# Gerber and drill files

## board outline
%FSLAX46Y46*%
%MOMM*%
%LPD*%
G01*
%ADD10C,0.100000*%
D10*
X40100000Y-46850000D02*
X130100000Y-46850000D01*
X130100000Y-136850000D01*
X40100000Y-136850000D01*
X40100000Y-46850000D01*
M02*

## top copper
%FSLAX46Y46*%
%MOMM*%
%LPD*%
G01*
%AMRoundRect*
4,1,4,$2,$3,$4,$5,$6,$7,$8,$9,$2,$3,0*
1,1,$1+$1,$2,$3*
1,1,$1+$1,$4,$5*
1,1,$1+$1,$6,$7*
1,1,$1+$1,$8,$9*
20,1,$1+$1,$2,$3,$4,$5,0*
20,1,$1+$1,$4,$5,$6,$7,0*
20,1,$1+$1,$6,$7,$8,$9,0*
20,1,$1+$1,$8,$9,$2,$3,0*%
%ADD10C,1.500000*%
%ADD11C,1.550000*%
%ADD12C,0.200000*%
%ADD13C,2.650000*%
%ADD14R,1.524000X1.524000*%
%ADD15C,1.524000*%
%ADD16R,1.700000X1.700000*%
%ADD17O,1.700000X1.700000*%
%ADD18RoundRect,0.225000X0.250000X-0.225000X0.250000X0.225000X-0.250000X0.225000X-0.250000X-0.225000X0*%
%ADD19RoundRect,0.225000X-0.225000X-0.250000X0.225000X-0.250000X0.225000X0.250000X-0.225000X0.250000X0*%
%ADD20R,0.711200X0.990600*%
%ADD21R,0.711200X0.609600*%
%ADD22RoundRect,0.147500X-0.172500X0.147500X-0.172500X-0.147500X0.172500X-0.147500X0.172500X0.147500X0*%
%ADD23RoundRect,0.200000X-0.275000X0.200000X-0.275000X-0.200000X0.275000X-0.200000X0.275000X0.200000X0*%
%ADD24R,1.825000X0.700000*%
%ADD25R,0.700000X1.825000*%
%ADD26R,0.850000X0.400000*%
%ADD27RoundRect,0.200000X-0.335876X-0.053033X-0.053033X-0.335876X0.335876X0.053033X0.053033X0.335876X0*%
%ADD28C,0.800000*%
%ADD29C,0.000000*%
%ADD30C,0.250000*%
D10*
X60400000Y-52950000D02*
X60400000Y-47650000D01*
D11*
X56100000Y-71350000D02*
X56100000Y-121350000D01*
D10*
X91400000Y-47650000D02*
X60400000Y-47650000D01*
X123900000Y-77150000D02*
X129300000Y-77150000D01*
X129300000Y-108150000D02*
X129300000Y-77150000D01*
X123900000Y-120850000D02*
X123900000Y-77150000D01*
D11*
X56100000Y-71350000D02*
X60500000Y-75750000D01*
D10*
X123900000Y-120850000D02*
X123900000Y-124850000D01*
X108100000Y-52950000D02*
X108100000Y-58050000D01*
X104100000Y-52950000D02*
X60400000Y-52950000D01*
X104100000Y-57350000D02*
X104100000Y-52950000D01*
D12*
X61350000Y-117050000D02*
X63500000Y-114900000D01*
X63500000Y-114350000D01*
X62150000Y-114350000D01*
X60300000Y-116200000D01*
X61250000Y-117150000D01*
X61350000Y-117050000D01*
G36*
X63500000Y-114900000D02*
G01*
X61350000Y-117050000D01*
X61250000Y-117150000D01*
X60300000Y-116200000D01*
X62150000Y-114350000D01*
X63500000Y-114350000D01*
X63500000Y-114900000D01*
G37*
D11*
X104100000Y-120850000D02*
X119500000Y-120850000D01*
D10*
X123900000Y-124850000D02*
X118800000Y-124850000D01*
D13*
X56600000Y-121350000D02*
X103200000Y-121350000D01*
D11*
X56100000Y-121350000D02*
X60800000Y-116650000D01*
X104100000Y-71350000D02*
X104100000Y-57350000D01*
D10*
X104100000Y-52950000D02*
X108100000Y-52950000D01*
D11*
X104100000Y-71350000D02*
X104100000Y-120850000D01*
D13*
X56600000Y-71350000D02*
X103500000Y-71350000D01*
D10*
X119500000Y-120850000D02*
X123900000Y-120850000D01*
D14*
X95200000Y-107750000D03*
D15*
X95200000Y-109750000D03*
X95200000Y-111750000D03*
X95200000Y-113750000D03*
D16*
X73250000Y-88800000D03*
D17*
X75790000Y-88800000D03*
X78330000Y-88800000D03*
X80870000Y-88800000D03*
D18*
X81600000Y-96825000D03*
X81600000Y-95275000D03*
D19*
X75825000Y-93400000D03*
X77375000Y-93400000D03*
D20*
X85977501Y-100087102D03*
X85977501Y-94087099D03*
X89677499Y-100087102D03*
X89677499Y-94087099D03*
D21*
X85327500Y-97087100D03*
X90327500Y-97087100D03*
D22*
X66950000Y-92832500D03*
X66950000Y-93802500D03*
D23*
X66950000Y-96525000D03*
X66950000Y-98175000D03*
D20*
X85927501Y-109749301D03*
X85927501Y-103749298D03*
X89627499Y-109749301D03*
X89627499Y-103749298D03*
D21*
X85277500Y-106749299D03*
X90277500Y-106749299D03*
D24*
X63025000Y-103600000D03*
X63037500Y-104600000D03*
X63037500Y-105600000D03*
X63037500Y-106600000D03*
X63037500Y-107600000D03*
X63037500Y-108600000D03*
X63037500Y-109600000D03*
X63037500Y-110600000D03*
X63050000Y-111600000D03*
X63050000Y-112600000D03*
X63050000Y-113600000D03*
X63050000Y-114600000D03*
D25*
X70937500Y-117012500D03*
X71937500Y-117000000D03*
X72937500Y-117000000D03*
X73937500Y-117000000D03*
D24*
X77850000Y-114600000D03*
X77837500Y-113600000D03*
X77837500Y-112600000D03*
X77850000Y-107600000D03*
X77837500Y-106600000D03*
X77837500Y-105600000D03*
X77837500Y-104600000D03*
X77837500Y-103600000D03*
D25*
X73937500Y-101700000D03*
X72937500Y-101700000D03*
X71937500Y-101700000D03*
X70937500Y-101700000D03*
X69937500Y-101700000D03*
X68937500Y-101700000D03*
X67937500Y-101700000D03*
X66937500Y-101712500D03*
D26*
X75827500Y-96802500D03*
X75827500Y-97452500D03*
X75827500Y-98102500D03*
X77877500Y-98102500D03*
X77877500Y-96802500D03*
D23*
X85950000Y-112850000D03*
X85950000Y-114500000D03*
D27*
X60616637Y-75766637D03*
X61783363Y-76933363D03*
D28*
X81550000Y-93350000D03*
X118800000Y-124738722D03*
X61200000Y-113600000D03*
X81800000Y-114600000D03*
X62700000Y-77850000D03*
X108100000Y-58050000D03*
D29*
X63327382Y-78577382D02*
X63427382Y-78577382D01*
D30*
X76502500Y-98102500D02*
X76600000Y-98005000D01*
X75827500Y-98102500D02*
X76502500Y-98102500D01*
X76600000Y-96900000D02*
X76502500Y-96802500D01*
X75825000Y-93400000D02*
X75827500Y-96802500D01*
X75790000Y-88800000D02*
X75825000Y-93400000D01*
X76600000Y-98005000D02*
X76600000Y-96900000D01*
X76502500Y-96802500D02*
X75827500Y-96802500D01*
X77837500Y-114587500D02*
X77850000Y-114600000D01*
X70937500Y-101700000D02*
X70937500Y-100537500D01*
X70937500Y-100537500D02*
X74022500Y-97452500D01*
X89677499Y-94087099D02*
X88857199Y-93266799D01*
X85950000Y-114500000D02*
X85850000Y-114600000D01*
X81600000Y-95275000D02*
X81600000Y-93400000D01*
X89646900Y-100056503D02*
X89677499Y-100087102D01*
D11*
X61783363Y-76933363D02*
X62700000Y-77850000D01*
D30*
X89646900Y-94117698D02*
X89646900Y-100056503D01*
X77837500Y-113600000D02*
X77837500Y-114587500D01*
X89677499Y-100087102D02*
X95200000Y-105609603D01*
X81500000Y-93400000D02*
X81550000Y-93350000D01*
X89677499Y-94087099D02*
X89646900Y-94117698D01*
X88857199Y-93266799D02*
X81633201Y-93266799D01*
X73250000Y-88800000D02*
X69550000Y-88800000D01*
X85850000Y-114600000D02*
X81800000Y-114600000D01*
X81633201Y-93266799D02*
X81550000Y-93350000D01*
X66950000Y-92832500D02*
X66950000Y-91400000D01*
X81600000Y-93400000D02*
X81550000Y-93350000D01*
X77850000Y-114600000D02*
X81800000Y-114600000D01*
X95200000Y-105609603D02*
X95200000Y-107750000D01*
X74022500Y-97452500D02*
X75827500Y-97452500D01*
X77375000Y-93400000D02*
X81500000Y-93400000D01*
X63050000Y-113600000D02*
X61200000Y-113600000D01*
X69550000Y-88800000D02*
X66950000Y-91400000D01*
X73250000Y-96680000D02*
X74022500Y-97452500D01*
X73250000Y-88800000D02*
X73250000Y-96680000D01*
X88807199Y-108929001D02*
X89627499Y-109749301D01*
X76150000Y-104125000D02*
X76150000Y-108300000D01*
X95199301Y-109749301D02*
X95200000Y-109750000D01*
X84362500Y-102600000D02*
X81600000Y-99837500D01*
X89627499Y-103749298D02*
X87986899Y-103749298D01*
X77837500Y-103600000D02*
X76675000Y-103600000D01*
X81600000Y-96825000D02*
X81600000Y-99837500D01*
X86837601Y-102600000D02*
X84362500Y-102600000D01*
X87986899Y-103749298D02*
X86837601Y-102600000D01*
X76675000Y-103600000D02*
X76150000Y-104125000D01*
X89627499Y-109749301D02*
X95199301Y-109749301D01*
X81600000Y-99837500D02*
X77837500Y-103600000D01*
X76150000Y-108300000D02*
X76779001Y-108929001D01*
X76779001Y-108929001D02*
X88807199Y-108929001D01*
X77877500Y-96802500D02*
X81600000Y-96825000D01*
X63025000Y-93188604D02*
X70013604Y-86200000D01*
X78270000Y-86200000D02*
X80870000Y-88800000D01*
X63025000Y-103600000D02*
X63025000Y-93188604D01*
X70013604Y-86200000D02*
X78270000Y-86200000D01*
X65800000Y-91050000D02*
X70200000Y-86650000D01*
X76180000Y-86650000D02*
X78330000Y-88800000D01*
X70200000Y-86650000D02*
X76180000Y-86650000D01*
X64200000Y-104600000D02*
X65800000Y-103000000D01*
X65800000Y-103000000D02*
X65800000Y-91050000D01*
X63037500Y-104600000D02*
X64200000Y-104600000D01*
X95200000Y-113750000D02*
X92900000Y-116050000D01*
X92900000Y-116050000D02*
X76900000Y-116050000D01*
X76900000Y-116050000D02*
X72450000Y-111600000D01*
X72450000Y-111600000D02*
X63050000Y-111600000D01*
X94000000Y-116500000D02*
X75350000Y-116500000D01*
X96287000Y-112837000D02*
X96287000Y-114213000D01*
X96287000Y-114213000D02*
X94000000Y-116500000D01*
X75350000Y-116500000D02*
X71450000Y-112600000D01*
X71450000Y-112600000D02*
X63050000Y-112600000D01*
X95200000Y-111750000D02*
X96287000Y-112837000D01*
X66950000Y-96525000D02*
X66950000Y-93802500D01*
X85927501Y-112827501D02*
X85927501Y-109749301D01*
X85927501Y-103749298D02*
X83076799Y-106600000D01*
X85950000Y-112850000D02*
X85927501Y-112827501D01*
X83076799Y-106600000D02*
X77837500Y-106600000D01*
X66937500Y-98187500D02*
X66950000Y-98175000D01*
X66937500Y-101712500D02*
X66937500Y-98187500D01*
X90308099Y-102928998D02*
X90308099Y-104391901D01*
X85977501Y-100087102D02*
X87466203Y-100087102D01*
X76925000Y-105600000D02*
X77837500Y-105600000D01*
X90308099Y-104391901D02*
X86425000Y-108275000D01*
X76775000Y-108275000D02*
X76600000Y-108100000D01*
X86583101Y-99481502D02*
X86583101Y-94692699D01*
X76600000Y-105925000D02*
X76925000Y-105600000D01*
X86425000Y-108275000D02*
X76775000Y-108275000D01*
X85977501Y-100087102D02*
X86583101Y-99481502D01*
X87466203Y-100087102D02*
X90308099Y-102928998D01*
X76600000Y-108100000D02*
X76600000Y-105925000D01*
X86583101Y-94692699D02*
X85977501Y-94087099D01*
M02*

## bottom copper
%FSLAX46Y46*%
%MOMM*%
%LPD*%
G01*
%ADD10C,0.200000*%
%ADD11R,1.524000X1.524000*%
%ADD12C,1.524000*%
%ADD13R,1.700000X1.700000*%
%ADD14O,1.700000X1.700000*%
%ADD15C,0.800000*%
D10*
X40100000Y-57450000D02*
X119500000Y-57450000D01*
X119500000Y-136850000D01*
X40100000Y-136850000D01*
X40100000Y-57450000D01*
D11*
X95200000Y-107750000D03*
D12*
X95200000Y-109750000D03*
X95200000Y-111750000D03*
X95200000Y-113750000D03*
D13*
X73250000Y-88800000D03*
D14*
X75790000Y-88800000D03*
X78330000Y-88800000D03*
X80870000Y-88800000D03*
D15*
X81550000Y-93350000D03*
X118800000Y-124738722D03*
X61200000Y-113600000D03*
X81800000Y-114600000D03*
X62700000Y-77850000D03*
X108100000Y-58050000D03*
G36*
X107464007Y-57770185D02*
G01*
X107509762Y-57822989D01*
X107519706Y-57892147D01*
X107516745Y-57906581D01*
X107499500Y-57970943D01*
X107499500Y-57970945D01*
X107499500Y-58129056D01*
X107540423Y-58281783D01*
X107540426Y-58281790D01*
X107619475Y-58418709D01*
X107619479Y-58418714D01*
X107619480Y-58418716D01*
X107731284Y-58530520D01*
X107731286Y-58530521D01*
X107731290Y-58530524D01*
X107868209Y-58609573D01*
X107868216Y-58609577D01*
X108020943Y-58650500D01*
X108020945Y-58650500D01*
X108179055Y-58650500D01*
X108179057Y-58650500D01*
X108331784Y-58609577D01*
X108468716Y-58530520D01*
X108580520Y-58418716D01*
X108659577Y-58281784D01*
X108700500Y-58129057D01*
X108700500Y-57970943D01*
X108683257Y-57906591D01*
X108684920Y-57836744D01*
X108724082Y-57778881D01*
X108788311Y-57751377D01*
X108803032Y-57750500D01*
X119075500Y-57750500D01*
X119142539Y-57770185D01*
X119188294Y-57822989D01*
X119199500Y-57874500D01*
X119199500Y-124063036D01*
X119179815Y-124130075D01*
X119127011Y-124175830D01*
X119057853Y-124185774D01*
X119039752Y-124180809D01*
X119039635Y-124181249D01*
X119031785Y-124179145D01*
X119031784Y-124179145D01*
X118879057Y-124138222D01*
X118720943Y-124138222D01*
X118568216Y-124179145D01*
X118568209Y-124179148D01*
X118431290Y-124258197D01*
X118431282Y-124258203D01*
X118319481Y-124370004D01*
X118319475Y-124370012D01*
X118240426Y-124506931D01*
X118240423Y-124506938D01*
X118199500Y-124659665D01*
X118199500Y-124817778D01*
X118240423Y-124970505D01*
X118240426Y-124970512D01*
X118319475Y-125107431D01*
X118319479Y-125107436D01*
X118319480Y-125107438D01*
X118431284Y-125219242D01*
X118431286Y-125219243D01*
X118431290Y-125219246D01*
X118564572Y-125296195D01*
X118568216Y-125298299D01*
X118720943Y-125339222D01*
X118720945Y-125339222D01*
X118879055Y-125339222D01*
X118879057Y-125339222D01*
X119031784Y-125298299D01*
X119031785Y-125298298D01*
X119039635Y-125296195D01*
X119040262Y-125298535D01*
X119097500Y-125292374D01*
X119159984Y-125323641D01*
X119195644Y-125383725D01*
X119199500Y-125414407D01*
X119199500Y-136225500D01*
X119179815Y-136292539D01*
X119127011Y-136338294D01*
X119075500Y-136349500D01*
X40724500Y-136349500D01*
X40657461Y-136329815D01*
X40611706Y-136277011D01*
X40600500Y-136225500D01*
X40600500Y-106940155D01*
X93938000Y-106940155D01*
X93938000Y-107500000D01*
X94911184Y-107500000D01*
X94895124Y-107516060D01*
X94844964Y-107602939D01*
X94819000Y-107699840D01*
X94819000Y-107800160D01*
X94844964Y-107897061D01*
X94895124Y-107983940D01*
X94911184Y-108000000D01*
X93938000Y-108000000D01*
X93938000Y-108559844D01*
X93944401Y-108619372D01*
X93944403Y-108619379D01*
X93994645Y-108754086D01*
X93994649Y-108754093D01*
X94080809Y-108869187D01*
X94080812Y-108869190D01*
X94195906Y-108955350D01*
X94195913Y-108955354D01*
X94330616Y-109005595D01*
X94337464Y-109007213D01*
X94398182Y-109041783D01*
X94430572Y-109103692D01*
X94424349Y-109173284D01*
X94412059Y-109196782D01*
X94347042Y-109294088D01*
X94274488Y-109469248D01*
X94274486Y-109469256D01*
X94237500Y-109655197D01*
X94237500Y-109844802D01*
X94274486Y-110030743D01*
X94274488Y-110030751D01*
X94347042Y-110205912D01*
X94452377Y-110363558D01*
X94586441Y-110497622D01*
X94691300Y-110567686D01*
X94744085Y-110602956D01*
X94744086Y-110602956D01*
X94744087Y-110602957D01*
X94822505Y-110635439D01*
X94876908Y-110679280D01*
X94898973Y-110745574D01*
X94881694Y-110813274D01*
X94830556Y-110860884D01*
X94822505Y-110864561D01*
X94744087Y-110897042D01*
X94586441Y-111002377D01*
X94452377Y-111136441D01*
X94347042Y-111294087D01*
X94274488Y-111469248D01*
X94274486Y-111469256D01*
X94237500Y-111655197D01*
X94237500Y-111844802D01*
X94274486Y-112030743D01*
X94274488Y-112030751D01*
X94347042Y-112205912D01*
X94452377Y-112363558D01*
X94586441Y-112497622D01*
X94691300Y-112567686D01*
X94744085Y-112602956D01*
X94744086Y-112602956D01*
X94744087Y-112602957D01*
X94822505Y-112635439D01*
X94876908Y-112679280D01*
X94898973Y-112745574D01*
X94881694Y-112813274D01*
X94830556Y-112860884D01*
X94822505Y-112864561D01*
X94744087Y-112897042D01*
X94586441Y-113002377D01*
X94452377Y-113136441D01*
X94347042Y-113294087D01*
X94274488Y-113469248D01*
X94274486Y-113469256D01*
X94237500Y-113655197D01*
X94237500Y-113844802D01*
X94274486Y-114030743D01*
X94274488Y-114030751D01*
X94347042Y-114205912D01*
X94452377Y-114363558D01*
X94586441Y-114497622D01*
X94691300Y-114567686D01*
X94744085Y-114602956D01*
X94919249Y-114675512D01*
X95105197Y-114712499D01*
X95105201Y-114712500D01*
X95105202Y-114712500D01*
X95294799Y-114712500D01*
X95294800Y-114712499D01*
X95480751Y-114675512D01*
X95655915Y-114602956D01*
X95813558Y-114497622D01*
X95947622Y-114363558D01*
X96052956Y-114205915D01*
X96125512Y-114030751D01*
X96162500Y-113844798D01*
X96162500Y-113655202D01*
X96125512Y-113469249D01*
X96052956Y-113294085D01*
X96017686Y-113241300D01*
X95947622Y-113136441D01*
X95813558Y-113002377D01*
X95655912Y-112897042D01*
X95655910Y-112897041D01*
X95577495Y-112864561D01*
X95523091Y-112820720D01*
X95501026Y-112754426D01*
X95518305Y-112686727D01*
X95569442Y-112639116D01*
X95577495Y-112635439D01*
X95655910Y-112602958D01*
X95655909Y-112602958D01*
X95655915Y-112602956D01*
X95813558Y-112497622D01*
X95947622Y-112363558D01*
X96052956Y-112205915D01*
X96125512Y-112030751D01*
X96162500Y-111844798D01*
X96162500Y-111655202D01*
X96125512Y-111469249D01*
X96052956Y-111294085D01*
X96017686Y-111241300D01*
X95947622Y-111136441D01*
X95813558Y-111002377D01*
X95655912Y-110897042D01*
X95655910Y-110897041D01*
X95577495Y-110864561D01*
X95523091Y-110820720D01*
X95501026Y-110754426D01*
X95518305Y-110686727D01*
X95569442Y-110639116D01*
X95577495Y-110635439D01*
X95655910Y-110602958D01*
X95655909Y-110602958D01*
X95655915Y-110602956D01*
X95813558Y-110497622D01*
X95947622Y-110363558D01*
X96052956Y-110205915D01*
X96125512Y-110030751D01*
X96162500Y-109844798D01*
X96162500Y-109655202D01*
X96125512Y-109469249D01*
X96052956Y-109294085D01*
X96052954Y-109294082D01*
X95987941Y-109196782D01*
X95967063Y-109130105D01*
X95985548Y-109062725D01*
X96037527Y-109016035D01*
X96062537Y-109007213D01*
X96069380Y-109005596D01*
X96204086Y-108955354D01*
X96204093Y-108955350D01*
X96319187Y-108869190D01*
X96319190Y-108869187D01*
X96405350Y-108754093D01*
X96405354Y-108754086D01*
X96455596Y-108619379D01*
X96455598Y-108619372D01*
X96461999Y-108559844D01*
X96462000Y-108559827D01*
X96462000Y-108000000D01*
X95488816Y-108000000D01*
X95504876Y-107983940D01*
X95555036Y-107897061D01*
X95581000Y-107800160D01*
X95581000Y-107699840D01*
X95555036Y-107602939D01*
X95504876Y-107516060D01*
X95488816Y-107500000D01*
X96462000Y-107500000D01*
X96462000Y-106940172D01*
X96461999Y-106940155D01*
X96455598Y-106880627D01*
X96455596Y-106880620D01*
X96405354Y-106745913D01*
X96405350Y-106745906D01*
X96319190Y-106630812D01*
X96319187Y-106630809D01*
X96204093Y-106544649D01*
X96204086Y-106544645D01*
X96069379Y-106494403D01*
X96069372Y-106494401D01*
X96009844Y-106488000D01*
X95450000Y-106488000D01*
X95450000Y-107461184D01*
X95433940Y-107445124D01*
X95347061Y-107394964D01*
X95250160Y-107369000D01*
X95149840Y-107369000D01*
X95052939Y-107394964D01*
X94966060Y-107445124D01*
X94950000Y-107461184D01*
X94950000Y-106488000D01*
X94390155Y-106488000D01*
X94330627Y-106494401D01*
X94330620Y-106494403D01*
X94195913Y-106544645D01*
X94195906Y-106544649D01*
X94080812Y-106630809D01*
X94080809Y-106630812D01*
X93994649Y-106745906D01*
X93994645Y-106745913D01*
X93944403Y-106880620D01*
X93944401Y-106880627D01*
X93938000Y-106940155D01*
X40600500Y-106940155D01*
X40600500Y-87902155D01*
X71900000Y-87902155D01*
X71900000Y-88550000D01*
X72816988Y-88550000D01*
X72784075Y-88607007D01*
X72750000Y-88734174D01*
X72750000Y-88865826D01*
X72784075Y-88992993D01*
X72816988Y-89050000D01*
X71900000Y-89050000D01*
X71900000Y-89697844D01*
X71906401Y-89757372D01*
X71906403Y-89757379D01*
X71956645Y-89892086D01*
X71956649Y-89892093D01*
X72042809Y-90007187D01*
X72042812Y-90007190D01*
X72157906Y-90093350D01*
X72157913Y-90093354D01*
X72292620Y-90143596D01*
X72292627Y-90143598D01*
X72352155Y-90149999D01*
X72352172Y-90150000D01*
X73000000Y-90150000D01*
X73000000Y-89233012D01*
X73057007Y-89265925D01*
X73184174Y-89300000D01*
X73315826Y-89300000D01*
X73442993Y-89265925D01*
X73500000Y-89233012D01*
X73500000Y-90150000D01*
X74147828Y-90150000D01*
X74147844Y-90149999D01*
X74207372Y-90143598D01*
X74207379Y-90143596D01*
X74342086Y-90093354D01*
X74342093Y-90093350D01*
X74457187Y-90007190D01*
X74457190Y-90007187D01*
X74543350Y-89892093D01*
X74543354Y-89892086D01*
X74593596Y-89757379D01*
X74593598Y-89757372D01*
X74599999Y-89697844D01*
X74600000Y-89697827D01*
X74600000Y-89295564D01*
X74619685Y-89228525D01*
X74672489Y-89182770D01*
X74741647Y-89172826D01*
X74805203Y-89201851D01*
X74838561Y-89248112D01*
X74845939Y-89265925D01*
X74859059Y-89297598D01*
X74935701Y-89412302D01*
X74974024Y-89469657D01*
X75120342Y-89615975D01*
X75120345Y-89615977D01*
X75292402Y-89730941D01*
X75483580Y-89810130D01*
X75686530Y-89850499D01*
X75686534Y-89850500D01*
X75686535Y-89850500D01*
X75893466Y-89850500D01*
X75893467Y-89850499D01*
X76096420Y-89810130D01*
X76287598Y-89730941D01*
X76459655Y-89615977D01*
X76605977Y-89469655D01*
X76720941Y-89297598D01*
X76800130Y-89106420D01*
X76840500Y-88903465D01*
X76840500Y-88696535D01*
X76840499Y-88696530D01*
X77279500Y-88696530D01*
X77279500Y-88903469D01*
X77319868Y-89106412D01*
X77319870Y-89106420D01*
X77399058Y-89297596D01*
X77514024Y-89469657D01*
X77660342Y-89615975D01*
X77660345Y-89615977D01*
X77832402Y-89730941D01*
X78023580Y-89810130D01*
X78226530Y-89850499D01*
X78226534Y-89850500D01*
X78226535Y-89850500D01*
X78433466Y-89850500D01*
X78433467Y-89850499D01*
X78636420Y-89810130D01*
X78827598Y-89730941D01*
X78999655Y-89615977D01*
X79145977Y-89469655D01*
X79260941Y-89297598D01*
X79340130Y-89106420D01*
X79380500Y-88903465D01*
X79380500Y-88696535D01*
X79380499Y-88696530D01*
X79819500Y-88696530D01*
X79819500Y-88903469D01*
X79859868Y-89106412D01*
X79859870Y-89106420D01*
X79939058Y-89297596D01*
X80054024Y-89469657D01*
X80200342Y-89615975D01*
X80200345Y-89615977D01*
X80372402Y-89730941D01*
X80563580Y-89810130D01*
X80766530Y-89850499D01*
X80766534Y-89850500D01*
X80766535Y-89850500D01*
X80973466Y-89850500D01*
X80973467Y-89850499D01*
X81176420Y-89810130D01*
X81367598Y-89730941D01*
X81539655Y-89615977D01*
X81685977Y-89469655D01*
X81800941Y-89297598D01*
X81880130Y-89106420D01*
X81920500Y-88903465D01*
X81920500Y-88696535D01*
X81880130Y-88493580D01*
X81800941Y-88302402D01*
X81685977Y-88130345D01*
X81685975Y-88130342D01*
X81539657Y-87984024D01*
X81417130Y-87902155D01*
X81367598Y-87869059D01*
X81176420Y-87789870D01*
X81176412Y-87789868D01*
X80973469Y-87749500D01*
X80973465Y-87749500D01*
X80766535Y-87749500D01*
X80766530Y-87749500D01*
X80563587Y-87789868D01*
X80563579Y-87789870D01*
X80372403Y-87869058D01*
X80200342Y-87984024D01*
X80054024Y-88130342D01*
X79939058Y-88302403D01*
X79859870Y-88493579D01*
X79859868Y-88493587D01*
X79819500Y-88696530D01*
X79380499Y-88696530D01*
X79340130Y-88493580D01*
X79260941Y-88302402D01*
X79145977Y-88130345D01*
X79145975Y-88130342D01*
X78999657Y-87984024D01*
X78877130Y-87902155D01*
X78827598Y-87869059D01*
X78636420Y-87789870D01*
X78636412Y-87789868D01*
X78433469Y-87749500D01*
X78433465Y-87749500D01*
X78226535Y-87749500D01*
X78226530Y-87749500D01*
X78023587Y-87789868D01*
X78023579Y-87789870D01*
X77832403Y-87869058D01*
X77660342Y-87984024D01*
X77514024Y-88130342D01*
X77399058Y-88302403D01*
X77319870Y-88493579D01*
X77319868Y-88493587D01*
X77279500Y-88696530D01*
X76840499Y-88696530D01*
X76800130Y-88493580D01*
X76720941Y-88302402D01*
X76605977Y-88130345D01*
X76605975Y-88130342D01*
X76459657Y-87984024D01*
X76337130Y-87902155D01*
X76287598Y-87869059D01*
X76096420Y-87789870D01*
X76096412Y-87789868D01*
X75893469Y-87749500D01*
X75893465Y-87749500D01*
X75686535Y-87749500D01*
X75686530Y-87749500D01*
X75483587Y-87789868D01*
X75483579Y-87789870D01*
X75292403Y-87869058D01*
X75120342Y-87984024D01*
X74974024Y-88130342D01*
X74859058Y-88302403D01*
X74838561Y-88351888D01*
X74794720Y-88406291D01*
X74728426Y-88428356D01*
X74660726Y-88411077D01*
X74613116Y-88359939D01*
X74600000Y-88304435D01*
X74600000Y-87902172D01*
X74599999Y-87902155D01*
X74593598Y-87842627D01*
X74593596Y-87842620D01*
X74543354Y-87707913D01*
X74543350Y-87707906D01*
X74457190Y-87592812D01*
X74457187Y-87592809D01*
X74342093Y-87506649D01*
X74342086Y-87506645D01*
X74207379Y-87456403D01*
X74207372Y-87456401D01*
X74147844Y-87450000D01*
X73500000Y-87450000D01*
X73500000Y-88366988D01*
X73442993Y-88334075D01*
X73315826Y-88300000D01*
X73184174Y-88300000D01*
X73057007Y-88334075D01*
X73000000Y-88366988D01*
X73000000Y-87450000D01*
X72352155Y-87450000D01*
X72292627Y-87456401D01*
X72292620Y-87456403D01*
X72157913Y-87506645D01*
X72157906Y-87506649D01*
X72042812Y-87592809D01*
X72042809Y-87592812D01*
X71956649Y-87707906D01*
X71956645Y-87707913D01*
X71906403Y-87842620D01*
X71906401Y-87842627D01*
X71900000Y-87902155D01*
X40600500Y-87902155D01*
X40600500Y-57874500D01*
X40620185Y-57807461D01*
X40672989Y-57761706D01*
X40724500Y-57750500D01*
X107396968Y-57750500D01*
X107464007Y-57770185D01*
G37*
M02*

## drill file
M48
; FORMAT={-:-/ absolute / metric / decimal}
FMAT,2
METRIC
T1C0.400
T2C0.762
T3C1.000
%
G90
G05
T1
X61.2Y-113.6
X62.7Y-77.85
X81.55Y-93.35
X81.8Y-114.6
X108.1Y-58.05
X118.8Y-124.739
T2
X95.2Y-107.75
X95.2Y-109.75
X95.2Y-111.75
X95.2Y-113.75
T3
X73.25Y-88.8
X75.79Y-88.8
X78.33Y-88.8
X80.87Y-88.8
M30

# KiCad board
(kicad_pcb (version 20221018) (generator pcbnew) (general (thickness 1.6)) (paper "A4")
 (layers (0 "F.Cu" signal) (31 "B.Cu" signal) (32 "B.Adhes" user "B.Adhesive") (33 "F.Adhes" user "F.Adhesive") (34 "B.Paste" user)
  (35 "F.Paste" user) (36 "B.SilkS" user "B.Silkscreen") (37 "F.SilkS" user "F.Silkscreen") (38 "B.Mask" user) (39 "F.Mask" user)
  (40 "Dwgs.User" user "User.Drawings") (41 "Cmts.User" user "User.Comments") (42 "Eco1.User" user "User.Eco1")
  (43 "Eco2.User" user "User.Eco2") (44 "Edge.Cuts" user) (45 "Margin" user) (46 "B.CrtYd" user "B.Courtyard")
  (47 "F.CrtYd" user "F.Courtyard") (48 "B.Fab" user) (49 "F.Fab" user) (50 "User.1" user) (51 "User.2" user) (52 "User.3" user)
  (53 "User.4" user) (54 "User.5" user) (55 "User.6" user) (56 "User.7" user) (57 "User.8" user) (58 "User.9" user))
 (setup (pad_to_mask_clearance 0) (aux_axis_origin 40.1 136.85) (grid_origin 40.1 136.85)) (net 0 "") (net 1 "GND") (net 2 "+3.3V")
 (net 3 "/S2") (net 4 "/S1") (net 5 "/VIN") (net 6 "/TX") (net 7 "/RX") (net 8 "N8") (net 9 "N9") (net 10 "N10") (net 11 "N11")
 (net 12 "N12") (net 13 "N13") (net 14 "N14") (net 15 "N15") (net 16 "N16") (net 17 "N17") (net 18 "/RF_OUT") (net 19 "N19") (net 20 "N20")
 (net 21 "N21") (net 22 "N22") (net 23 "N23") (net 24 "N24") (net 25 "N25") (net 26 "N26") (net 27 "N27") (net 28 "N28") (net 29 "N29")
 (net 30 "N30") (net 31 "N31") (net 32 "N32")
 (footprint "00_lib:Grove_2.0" (layer "F.Cu") (at 95.05 110.75)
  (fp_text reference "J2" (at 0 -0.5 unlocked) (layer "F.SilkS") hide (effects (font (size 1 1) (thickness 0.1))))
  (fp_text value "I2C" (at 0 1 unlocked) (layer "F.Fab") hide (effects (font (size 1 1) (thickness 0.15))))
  (pad "1" thru_hole rect (at 0.15 -3) (size 1.524 1.524) (drill 0.762) (layers "*.Cu" "*.Mask") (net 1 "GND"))
  (pad "2" thru_hole circle (at 0.15 -1) (size 1.524 1.524) (drill 0.762) (layers "*.Cu" "*.Mask") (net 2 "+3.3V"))
  (pad "3" thru_hole circle (at 0.15 1) (size 1.524 1.524) (drill 0.762) (layers "*.Cu" "*.Mask") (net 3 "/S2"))
  (pad "4" thru_hole circle (at 0.15 3) (size 1.524 1.524) (drill 0.762) (layers "*.Cu" "*.Mask") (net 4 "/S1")))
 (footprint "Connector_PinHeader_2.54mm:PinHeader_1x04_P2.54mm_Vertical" (layer "F.Cu") (at 73.25 88.8 90)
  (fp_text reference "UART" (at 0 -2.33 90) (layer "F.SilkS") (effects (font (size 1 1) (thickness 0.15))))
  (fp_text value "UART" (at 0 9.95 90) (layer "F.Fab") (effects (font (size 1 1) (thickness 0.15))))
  (pad "1" thru_hole rect (at 0 0 90) (size 1.7 1.7) (drill 1) (layers "*.Cu" "*.Mask") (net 1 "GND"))
  (pad "2" thru_hole oval (at 0 2.54 90) (size 1.7 1.7) (drill 1) (layers "*.Cu" "*.Mask") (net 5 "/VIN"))
  (pad "3" thru_hole oval (at 0 5.08 90) (size 1.7 1.7) (drill 1) (layers "*.Cu" "*.Mask") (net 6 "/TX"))
  (pad "4" thru_hole oval (at 0 7.62 90) (size 1.7 1.7) (drill 1) (layers "*.Cu" "*.Mask") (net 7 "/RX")))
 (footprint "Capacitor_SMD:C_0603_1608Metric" (layer "F.Cu") (at 81.6 96.05 90)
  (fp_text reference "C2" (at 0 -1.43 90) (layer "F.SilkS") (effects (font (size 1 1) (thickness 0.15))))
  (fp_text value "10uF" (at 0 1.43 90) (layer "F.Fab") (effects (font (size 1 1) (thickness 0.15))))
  (pad "1" smd roundrect (at -0.775 0 90) (size 0.9 0.95) (layers "F.Cu" "F.Paste" "F.Mask") (roundrect_rratio 0.25) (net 2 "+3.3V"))
  (pad "2" smd roundrect (at 0.775 0 90) (size 0.9 0.95) (layers "F.Cu" "F.Paste" "F.Mask") (roundrect_rratio 0.25) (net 1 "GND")))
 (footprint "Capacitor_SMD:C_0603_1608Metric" (layer "F.Cu") (at 76.6 93.4)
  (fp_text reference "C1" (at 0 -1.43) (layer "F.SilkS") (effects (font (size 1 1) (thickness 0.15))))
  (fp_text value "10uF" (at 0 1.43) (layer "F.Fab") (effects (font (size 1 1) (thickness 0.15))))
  (pad "1" smd roundrect (at -0.775 0) (size 0.9 0.95) (layers "F.Cu" "F.Paste" "F.Mask") (roundrect_rratio 0.25) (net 5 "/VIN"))
  (pad "2" smd roundrect (at 0.775 0) (size 0.9 0.95) (layers "F.Cu" "F.Paste" "F.Mask") (roundrect_rratio 0.25) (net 1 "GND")))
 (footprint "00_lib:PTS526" (layer "F.Cu") (at 87.7363 97.037801 90)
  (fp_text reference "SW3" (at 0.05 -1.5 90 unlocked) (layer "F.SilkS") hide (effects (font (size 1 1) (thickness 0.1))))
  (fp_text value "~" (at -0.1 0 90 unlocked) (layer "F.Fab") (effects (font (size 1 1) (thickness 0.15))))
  (pad "1" smd rect (at -3.049301 -1.758799 90) (size 0.9906 0.7112) (layers "F.Cu" "F.Paste" "F.Mask") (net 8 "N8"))
  (pad "2" smd rect (at 2.950702 -1.758799 90) (size 0.9906 0.7112) (layers "F.Cu" "F.Paste" "F.Mask") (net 8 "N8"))
  (pad "3" smd rect (at -3.049301 1.941199 90) (size 0.9906 0.7112) (layers "F.Cu" "F.Paste" "F.Mask") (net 1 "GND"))
  (pad "4" smd rect (at 2.950702 1.941199 90) (size 0.9906 0.7112) (layers "F.Cu" "F.Paste" "F.Mask") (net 1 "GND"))
  (pad "5" smd rect (at -0.049299 -2.4088 180) (size 0.7112 0.6096) (layers "F.Cu" "F.Paste" "F.Mask"))
  (pad "6" smd rect (at -0.049299 2.5912 180) (size 0.7112 0.6096) (layers "F.Cu" "F.Paste" "F.Mask")))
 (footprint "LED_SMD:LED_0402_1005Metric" (layer "F.Cu") (at 66.95 93.3175 -90)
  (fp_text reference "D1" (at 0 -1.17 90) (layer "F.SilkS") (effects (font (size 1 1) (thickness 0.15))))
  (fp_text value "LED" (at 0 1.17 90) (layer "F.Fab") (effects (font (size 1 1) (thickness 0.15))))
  (pad "1" smd roundrect (at -0.485 0 270) (size 0.59 0.64) (layers "F.Cu" "F.Paste" "F.Mask") (roundrect_rratio 0.25) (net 1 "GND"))
  (pad "2" smd roundrect (at 0.485 0 270) (size 0.59 0.64) (layers "F.Cu" "F.Paste" "F.Mask") (roundrect_rratio 0.25) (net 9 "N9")))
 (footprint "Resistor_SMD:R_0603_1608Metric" (layer "F.Cu") (at 66.95 97.35 -90)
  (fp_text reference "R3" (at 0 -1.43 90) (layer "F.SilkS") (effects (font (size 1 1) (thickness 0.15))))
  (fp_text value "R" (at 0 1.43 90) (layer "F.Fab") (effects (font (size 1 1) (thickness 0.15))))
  (pad "1" smd roundrect (at -0.825 0 270) (size 0.8 0.95) (layers "F.Cu" "F.Paste" "F.Mask") (roundrect_rratio 0.25) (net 9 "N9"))
  (pad "2" smd roundrect (at 0.825 0 270) (size 0.8 0.95) (layers "F.Cu" "F.Paste" "F.Mask") (roundrect_rratio 0.25) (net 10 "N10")))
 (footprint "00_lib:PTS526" (layer "F.Cu") (at 87.6863 106.7 90)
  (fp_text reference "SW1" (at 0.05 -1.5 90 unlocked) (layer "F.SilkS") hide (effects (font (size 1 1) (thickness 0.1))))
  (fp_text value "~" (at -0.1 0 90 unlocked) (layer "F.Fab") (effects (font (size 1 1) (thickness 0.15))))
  (pad "1" smd rect (at -3.049301 -1.758799 90) (size 0.9906 0.7112) (layers "F.Cu" "F.Paste" "F.Mask") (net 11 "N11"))
  (pad "2" smd rect (at 2.950702 -1.758799 90) (size 0.9906 0.7112) (layers "F.Cu" "F.Paste" "F.Mask") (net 11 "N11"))
  (pad "3" smd rect (at -3.049301 1.941199 90) (size 0.9906 0.7112) (layers "F.Cu" "F.Paste" "F.Mask") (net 2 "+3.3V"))
  (pad "4" smd rect (at 2.950702 1.941199 90) (size 0.9906 0.7112) (layers "F.Cu" "F.Paste" "F.Mask") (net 2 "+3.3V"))
  (pad "5" smd rect (at -0.049299 -2.4088 180) (size 0.7112 0.6096) (layers "F.Cu" "F.Paste" "F.Mask"))
  (pad "6" smd rect (at -0.049299 2.5912 180) (size 0.7112 0.6096) (layers "F.Cu" "F.Paste" "F.Mask")))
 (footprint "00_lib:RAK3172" (layer "F.Cu") (at 70.4875 109.35 90)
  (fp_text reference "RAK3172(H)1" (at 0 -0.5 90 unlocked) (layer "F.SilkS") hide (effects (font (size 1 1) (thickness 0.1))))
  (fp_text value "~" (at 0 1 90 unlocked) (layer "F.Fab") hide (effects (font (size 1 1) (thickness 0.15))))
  (pad "1" smd rect (at 5.75 -7.4625 180) (size 1.825 0.7) (layers "F.Cu" "F.Paste" "F.Mask") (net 7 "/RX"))
  (pad "2" smd rect (at 4.75 -7.45 180) (size 1.825 0.7) (layers "F.Cu" "F.Paste" "F.Mask") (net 6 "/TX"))
  (pad "3" smd rect (at 3.75 -7.45 180) (size 1.825 0.7) (layers "F.Cu" "F.Paste" "F.Mask") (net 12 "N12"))
  (pad "4" smd rect (at 2.75 -7.45 180) (size 1.825 0.7) (layers "F.Cu" "F.Paste" "F.Mask") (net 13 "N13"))
  (pad "5" smd rect (at 1.75 -7.45 180) (size 1.825 0.7) (layers "F.Cu" "F.Paste" "F.Mask") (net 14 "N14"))
  (pad "6" smd rect (at 0.75 -7.45 180) (size 1.825 0.7) (layers "F.Cu" "F.Paste" "F.Mask") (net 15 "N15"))
  (pad "7" smd rect (at -0.25 -7.45 180) (size 1.825 0.7) (layers "F.Cu" "F.Paste" "F.Mask") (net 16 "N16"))
  (pad "8" smd rect (at -1.25 -7.45 180) (size 1.825 0.7) (layers "F.Cu" "F.Paste" "F.Mask") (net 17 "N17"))
  (pad "9" smd rect (at -2.25 -7.4375 180) (size 1.825 0.7) (layers "F.Cu" "F.Paste" "F.Mask") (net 4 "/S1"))
  (pad "10" smd rect (at -3.25 -7.4375 180) (size 1.825 0.7) (layers "F.Cu" "F.Paste" "F.Mask") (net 3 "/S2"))
  (pad "11" smd rect (at -4.25 -7.4375 180) (size 1.825 0.7) (layers "F.Cu" "F.Paste" "F.Mask") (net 1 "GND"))
  (pad "12" smd rect (at -5.25 -7.4375 180) (size 1.825 0.7) (layers "F.Cu" "F.Paste" "F.Mask") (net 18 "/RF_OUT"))
  (pad "13" smd rect (at -7.6625 0.45 270) (size 1.825 0.7) (layers "F.Cu" "F.Paste" "F.Mask") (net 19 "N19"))
  (pad "14" smd rect (at -7.65 1.45 270) (size 1.825 0.7) (layers "F.Cu" "F.Paste" "F.Mask") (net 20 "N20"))
  (pad "15" smd rect (at -7.65 2.45 270) (size 1.825 0.7) (layers "F.Cu" "F.Paste" "F.Mask") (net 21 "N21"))
  (pad "16" smd rect (at -7.65 3.45 270) (size 1.825 0.7) (layers "F.Cu" "F.Paste" "F.Mask") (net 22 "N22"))
  (pad "17" smd rect (at -5.25 7.3625) (size 1.825 0.7) (layers "F.Cu" "F.Paste" "F.Mask") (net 1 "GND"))
  (pad "18" smd rect (at -4.25 7.35) (size 1.825 0.7) (layers "F.Cu" "F.Paste" "F.Mask") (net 1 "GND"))
  (pad "19" smd rect (at -3.25 7.35) (size 1.825 0.7) (layers "F.Cu" "F.Paste" "F.Mask") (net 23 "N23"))
  (pad "20" smd rect (at 1.75 7.3625) (size 1.825 0.7) (layers "F.Cu" "F.Paste" "F.Mask") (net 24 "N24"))
  (pad "21" smd rect (at 2.75 7.35) (size 1.825 0.7) (layers "F.Cu" "F.Paste" "F.Mask") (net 11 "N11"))
  (pad "22" smd rect (at 3.75 7.35) (size 1.825 0.7) (layers "F.Cu" "F.Paste" "F.Mask") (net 8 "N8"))
  (pad "23" smd rect (at 4.75 7.35) (size 1.825 0.7) (layers "F.Cu" "F.Paste" "F.Mask") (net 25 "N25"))
  (pad "24" smd rect (at 5.75 7.35) (size 1.825 0.7) (layers "F.Cu" "F.Paste" "F.Mask") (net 2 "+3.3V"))
  (pad "25" smd rect (at 7.65 3.45 270) (size 1.825 0.7) (layers "F.Cu" "F.Paste" "F.Mask") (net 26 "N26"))
  (pad "26" smd rect (at 7.65 2.45 270) (size 1.825 0.7) (layers "F.Cu" "F.Paste" "F.Mask") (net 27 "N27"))
  (pad "27" smd rect (at 7.65 1.45 270) (size 1.825 0.7) (layers "F.Cu" "F.Paste" "F.Mask") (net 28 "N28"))
  (pad "28" smd rect (at 7.65 0.45 270) (size 1.825 0.7) (layers "F.Cu" "F.Paste" "F.Mask") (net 1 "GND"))
  (pad "29" smd rect (at 7.65 -0.55 270) (size 1.825 0.7) (layers "F.Cu" "F.Paste" "F.Mask") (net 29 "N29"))
  (pad "30" smd rect (at 7.65 -1.55 270) (size 1.825 0.7) (layers "F.Cu" "F.Paste" "F.Mask") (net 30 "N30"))
  (pad "31" smd rect (at 7.65 -2.55 270) (size 1.825 0.7) (layers "F.Cu" "F.Paste" "F.Mask") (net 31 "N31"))
  (pad "32" smd rect (at 7.6375 -3.55 270) (size 1.825 0.7) (layers "F.Cu" "F.Paste" "F.Mask") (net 10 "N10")))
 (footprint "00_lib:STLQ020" (layer "F.Cu") (at 76.9025 97.5025)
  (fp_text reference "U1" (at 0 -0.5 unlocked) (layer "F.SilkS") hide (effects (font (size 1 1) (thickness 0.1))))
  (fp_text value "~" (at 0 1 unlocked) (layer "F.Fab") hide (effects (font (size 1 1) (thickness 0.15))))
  (pad "1" smd rect (at -1.075 -0.7) (size 0.85 0.4) (layers "F.Cu" "F.Paste" "F.Mask") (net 5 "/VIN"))
  (pad "2" smd rect (at -1.075 -0.05) (size 0.85 0.4) (layers "F.Cu" "F.Paste" "F.Mask") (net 1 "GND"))
  (pad "3" smd rect (at -1.075 0.6) (size 0.85 0.4) (layers "F.Cu" "F.Paste" "F.Mask") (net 5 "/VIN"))
  (pad "4" smd rect (at 0.975 0.6) (size 0.85 0.4) (layers "F.Cu" "F.Paste" "F.Mask") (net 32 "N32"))
  (pad "5" smd rect (at 0.975 -0.7) (size 0.85 0.4) (layers "F.Cu" "F.Paste" "F.Mask") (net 2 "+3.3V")))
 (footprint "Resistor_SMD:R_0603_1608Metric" (layer "F.Cu") (at 85.95 113.675 -90)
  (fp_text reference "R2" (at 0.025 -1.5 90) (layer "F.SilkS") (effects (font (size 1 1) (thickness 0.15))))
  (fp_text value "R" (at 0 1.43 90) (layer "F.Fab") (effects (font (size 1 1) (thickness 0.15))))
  (pad "1" smd roundrect (at -0.825 0 270) (size 0.8 0.95) (layers "F.Cu" "F.Paste" "F.Mask") (roundrect_rratio 0.25) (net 11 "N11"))
  (pad "2" smd roundrect (at 0.825 0 270) (size 0.8 0.95) (layers "F.Cu" "F.Paste" "F.Mask") (roundrect_rratio 0.25) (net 1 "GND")))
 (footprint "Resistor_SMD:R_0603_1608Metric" (layer "F.Cu") (at 61.2 76.35 -45)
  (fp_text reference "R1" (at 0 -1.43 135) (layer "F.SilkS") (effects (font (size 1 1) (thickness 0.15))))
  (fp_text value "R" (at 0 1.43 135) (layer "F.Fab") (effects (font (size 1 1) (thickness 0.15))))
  (pad "1" smd roundrect (at -0.825 0 315) (size 0.8 0.95) (layers "F.Cu" "F.Paste" "F.Mask") (roundrect_rratio 0.25) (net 18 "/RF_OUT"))
  (pad "2" smd roundrect (at 0.825 0 315) (size 0.8 0.95) (layers "F.Cu" "F.Paste" "F.Mask") (roundrect_rratio 0.25) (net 1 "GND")))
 (gr_line (start 60.4 52.95) (end 60.4 47.65) (stroke (width 1.5) (type default)) (layer "F.Cu"))
 (gr_line (start 56.1 71.35) (end 56.1 121.35) (stroke (width 1.55) (type default)) (layer "F.Cu"))
 (gr_line (start 91.4 47.65) (end 60.4 47.65) (stroke (width 1.5) (type default)) (layer "F.Cu"))
 (gr_line (start 123.9 77.15) (end 129.3 77.15) (stroke (width 1.5) (type default)) (layer "F.Cu"))
 (gr_line (start 129.3 108.15) (end 129.3 77.15) (stroke (width 1.5) (type default)) (layer "F.Cu"))
 (gr_line (start 123.9 120.85) (end 123.9 77.15) (stroke (width 1.5) (type default)) (layer "F.Cu"))
 (gr_line (start 56.1 71.35) (end 60.5 75.75) (stroke (width 1.55) (type default)) (layer "F.Cu"))
 (gr_line (start 123.9 120.85) (end 123.9 124.85) (stroke (width 1.5) (type default)) (layer "F.Cu"))
 (gr_line (start 108.1 52.95) (end 108.1 58.05) (stroke (width 1.5) (type default)) (layer "F.Cu"))
 (gr_line (start 104.1 52.95) (end 60.4 52.95) (stroke (width 1.5) (type default)) (layer "F.Cu"))
 (gr_line (start 104.1 57.35) (end 104.1 52.95) (stroke (width 1.5) (type default)) (layer "F.Cu"))
 (gr_poly
  (pts (xy 61.35 117.05) (xy 63.5 114.9) (xy 63.5 114.35) (xy 62.15 114.35) (xy 60.3 116.2) (xy 61.25 117.15))
  (stroke (width 0.2) (type solid)) (fill solid) (layer "F.Cu"))
 (gr_line (start 104.1 120.85) (end 119.5 120.85) (stroke (width 1.55) (type default)) (layer "F.Cu"))
 (gr_line (start 123.9 124.85) (end 118.8 124.85) (stroke (width 1.5) (type default)) (layer "F.Cu"))
 (gr_line (start 56.6 121.35) (end 103.2 121.35) (stroke (width 2.65) (type default)) (layer "F.Cu"))
 (gr_line (start 56.1 121.35) (end 60.8 116.65) (stroke (width 1.55) (type default)) (layer "F.Cu"))
 (gr_line (start 104.1 71.35) (end 104.1 57.35) (stroke (width 1.55) (type default)) (layer "F.Cu"))
 (gr_line (start 104.1 52.95) (end 108.1 52.95) (stroke (width 1.5) (type default)) (layer "F.Cu"))
 (gr_line (start 104.1 71.35) (end 104.1 120.85) (stroke (width 1.55) (type default)) (layer "F.Cu"))
 (gr_line (start 56.6 71.35) (end 103.5 71.35) (stroke (width 2.65) (type default)) (layer "F.Cu"))
 (gr_line (start 119.5 120.85) (end 123.9 120.85) (stroke (width 1.5) (type default)) (layer "F.Cu"))
 (gr_rect (start 40.1 57.45) (end 119.5 136.85) (stroke (width 0.2) (type default)) (fill none) (layer "B.Cu"))
 (gr_rect (start 40.1 46.85) (end 130.1 136.85) (stroke (width 0.1) (type default)) (fill none) (layer "Edge.Cuts"))
 (segment (start 63.327382 78.577382) (end 63.427382 78.577382) (width 0) (layer "F.Cu") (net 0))
 (segment (start 76.5025 98.1025) (end 76.6 98.005) (width 0.25) (layer "F.Cu") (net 5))
 (segment (start 75.8275 98.1025) (end 76.5025 98.1025) (width 0.25) (layer "F.Cu") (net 5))
 (segment (start 76.6 96.9) (end 76.5025 96.8025) (width 0.25) (layer "F.Cu") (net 5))
 (segment (start 75.825 93.4) (end 75.8275 96.8025) (width 0.25) (layer "F.Cu") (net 5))
 (segment (start 75.79 88.8) (end 75.825 93.4) (width 0.25) (layer "F.Cu") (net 5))
 (segment (start 76.6 98.005) (end 76.6 96.9) (width 0.25) (layer "F.Cu") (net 5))
 (segment (start 76.5025 96.8025) (end 75.8275 96.8025) (width 0.25) (layer "F.Cu") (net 5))
 (segment (start 77.8375 114.5875) (end 77.85 114.6) (width 0.25) (layer "F.Cu") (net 1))
 (segment (start 70.9375 101.7) (end 70.9375 100.5375) (width 0.25) (layer "F.Cu") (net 1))
 (segment (start 70.9375 100.5375) (end 74.0225 97.4525) (width 0.25) (layer "F.Cu") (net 1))
 (segment (start 89.677499 94.087099) (end 88.857199 93.266799) (width 0.25) (layer "F.Cu") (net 1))
 (segment (start 85.95 114.5) (end 85.85 114.6) (width 0.25) (layer "F.Cu") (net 1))
 (segment (start 81.6 95.275) (end 81.6 93.4) (width 0.25) (layer "F.Cu") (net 1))
 (segment (start 89.6469 100.056503) (end 89.677499 100.087102) (width 0.25) (layer "F.Cu") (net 1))
 (segment (start 61.783363 76.933363) (end 62.7 77.85) (width 1.55) (layer "F.Cu") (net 1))
 (segment (start 89.6469 94.117698) (end 89.6469 100.056503) (width 0.25) (layer "F.Cu") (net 1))
 (segment (start 77.8375 113.6) (end 77.8375 114.5875) (width 0.25) (layer "F.Cu") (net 1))
 (segment (start 89.677499 100.087102) (end 95.2 105.609603) (width 0.25) (layer "F.Cu") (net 1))
 (segment (start 81.5 93.4) (end 81.55 93.35) (width 0.25) (layer "F.Cu") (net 1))
 (segment (start 89.677499 94.087099) (end 89.6469 94.117698) (width 0.25) (layer "F.Cu") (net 1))
 (segment (start 88.857199 93.266799) (end 81.633201 93.266799) (width 0.25) (layer "F.Cu") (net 1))
 (segment (start 73.25 88.8) (end 69.55 88.8) (width 0.25) (layer "F.Cu") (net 1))
 (segment (start 85.85 114.6) (end 81.8 114.6) (width 0.25) (layer "F.Cu") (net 1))
 (segment (start 81.633201 93.266799) (end 81.55 93.35) (width 0.25) (layer "F.Cu") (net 1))
 (segment (start 66.95 92.8325) (end 66.95 91.4) (width 0.25) (layer "F.Cu") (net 1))
 (segment (start 81.6 93.4) (end 81.55 93.35) (width 0.25) (layer "F.Cu") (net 1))
 (segment (start 77.85 114.6) (end 81.8 114.6) (width 0.25) (layer "F.Cu") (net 1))
 (segment (start 95.2 105.609603) (end 95.2 107.75) (width 0.25) (layer "F.Cu") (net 1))
 (segment (start 74.0225 97.4525) (end 75.8275 97.4525) (width 0.25) (layer "F.Cu") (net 1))
 (segment (start 77.375 93.4) (end 81.5 93.4) (width 0.25) (layer "F.Cu") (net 1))
 (segment (start 63.05 113.6) (end 61.2 113.6) (width 0.25) (layer "F.Cu") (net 1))
 (segment (start 69.55 88.8) (end 66.95 91.4) (width 0.25) (layer "F.Cu") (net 1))
 (segment (start 73.25 96.68) (end 74.0225 97.4525) (width 0.25) (layer "F.Cu") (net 1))
 (segment (start 73.25 88.8) (end 73.25 96.68) (width 0.25) (layer "F.Cu") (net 1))
 (via (at 81.55 93.35) (size 0.8) (drill 0.4) (layers "F.Cu" "B.Cu") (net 1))
 (via (at 118.8 124.738722) (size 0.8) (drill 0.4) (layers "F.Cu" "B.Cu") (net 1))
 (via (at 61.2 113.6) (size 0.8) (drill 0.4) (layers "F.Cu" "B.Cu") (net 1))
 (via (at 81.8 114.6) (size 0.8) (drill 0.4) (layers "F.Cu" "B.Cu") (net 1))
 (via (at 62.7 77.85) (size 0.8) (drill 0.4) (layers "F.Cu" "B.Cu") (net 1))
 (via (at 108.1 58.05) (size 0.8) (drill 0.4) (layers "F.Cu" "B.Cu") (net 1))
 (segment (start 88.807199 108.929001) (end 89.627499 109.749301) (width 0.25) (layer "F.Cu") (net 2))
 (segment (start 76.15 104.125) (end 76.15 108.3) (width 0.25) (layer "F.Cu") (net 2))
 (segment (start 95.199301 109.749301) (end 95.2 109.75) (width 0.25) (layer "F.Cu") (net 2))
 (segment (start 84.3625 102.6) (end 81.6 99.8375) (width 0.25) (layer "F.Cu") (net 2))
 (segment (start 89.627499 103.749298) (end 87.986899 103.749298) (width 0.25) (layer "F.Cu") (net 2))
 (segment (start 77.8375 103.6) (end 76.675 103.6) (width 0.25) (layer "F.Cu") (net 2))
 (segment (start 81.6 96.825) (end 81.6 99.8375) (width 0.25) (layer "F.Cu") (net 2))
 (segment (start 86.837601 102.6) (end 84.3625 102.6) (width 0.25) (layer "F.Cu") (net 2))
 (segment (start 87.986899 103.749298) (end 86.837601 102.6) (width 0.25) (layer "F.Cu") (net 2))
 (segment (start 76.675 103.6) (end 76.15 104.125) (width 0.25) (layer "F.Cu") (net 2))
 (segment (start 89.627499 109.749301) (end 95.199301 109.749301) (width 0.25) (layer "F.Cu") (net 2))
 (segment (start 81.6 99.8375) (end 77.8375 103.6) (width 0.25) (layer "F.Cu") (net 2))
 (segment (start 76.15 108.3) (end 76.779001 108.929001) (width 0.25) (layer "F.Cu") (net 2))
 (segment (start 76.779001 108.929001) (end 88.807199 108.929001) (width 0.25) (layer "F.Cu") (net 2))
 (segment (start 77.8775 96.8025) (end 81.6 96.825) (width 0.25) (layer "F.Cu") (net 2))
 (segment (start 63.025 93.188604) (end 70.013604 86.2) (width 0.25) (layer "F.Cu") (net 7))
 (segment (start 78.27 86.2) (end 80.87 88.8) (width 0.25) (layer "F.Cu") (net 7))
 (segment (start 63.025 103.6) (end 63.025 93.188604) (width 0.25) (layer "F.Cu") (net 7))
 (segment (start 70.013604 86.2) (end 78.27 86.2) (width 0.25) (layer "F.Cu") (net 7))
 (segment (start 65.8 91.05) (end 70.2 86.65) (width 0.25) (layer "F.Cu") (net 6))
 (segment (start 76.18 86.65) (end 78.33 88.8) (width 0.25) (layer "F.Cu") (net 6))
 (segment (start 70.2 86.65) (end 76.18 86.65) (width 0.25) (layer "F.Cu") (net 6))
 (segment (start 64.2 104.6) (end 65.8 103) (width 0.25) (layer "F.Cu") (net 6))
 (segment (start 65.8 103) (end 65.8 91.05) (width 0.25) (layer "F.Cu") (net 6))
 (segment (start 63.0375 104.6) (end 64.2 104.6) (width 0.25) (layer "F.Cu") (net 6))
 (segment (start 95.2 113.75) (end 92.9 116.05) (width 0.25) (layer "F.Cu") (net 4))
 (segment (start 92.9 116.05) (end 76.9 116.05) (width 0.25) (layer "F.Cu") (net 4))
 (segment (start 76.9 116.05) (end 72.45 111.6) (width 0.25) (layer "F.Cu") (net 4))
 (segment (start 72.45 111.6) (end 63.05 111.6) (width 0.25) (layer "F.Cu") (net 4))
 (segment (start 94 116.5) (end 75.35 116.5) (width 0.25) (layer "F.Cu") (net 3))
 (segment (start 96.287 112.837) (end 96.287 114.213) (width 0.25) (layer "F.Cu") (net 3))
 (segment (start 96.287 114.213) (end 94 116.5) (width 0.25) (layer "F.Cu") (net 3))
 (segment (start 75.35 116.5) (end 71.45 112.6) (width 0.25) (layer "F.Cu") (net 3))
 (segment (start 71.45 112.6) (end 63.05 112.6) (width 0.25) (layer "F.Cu") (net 3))
 (segment (start 95.2 111.75) (end 96.287 112.837) (width 0.25) (layer "F.Cu") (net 3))
 (segment (start 66.95 96.525) (end 66.95 93.8025) (width 0.25) (layer "F.Cu") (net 9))
 (segment (start 85.927501 112.827501) (end 85.927501 109.749301) (width 0.25) (layer "F.Cu") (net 11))
 (segment (start 85.927501 103.749298) (end 83.076799 106.6) (width 0.25) (layer "F.Cu") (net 11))
 (segment (start 85.95 112.85) (end 85.927501 112.827501) (width 0.25) (layer "F.Cu") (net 11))
 (segment (start 83.076799 106.6) (end 77.8375 106.6) (width 0.25) (layer "F.Cu") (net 11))
 (segment (start 66.9375 98.1875) (end 66.95 98.175) (width 0.25) (layer "F.Cu") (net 10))
 (segment (start 66.9375 101.7125) (end 66.9375 98.1875) (width 0.25) (layer "F.Cu") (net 10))
 (segment (start 90.308099 102.928998) (end 90.308099 104.391901) (width 0.25) (layer "F.Cu") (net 8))
 (segment (start 85.977501 100.087102) (end 87.466203 100.087102) (width 0.25) (layer "F.Cu") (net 8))
 (segment (start 76.925 105.6) (end 77.8375 105.6) (width 0.25) (layer "F.Cu") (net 8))
 (segment (start 90.308099 104.391901) (end 86.425 108.275) (width 0.25) (layer "F.Cu") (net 8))
 (segment (start 76.775 108.275) (end 76.6 108.1) (width 0.25) (layer "F.Cu") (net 8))
 (segment (start 86.583101 99.481502) (end 86.583101 94.692699) (width 0.25) (layer "F.Cu") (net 8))
 (segment (start 76.6 105.925) (end 76.925 105.6) (width 0.25) (layer "F.Cu") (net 8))
 (segment (start 86.425 108.275) (end 76.775 108.275) (width 0.25) (layer "F.Cu") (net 8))
 (segment (start 85.977501 100.087102) (end 86.583101 99.481502) (width 0.25) (layer "F.Cu") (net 8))
 (segment (start 87.466203 100.087102) (end 90.308099 102.928998) (width 0.25) (layer "F.Cu") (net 8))
 (segment (start 76.6 108.1) (end 76.6 105.925) (width 0.25) (layer "F.Cu") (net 8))
 (segment (start 86.583101 94.692699) (end 85.977501 94.087099) (width 0.25) (layer "F.Cu") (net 8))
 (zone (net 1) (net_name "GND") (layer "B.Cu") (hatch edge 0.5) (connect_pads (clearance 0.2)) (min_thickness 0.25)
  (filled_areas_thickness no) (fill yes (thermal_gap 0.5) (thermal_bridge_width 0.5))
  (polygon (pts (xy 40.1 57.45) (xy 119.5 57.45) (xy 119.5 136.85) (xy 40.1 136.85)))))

